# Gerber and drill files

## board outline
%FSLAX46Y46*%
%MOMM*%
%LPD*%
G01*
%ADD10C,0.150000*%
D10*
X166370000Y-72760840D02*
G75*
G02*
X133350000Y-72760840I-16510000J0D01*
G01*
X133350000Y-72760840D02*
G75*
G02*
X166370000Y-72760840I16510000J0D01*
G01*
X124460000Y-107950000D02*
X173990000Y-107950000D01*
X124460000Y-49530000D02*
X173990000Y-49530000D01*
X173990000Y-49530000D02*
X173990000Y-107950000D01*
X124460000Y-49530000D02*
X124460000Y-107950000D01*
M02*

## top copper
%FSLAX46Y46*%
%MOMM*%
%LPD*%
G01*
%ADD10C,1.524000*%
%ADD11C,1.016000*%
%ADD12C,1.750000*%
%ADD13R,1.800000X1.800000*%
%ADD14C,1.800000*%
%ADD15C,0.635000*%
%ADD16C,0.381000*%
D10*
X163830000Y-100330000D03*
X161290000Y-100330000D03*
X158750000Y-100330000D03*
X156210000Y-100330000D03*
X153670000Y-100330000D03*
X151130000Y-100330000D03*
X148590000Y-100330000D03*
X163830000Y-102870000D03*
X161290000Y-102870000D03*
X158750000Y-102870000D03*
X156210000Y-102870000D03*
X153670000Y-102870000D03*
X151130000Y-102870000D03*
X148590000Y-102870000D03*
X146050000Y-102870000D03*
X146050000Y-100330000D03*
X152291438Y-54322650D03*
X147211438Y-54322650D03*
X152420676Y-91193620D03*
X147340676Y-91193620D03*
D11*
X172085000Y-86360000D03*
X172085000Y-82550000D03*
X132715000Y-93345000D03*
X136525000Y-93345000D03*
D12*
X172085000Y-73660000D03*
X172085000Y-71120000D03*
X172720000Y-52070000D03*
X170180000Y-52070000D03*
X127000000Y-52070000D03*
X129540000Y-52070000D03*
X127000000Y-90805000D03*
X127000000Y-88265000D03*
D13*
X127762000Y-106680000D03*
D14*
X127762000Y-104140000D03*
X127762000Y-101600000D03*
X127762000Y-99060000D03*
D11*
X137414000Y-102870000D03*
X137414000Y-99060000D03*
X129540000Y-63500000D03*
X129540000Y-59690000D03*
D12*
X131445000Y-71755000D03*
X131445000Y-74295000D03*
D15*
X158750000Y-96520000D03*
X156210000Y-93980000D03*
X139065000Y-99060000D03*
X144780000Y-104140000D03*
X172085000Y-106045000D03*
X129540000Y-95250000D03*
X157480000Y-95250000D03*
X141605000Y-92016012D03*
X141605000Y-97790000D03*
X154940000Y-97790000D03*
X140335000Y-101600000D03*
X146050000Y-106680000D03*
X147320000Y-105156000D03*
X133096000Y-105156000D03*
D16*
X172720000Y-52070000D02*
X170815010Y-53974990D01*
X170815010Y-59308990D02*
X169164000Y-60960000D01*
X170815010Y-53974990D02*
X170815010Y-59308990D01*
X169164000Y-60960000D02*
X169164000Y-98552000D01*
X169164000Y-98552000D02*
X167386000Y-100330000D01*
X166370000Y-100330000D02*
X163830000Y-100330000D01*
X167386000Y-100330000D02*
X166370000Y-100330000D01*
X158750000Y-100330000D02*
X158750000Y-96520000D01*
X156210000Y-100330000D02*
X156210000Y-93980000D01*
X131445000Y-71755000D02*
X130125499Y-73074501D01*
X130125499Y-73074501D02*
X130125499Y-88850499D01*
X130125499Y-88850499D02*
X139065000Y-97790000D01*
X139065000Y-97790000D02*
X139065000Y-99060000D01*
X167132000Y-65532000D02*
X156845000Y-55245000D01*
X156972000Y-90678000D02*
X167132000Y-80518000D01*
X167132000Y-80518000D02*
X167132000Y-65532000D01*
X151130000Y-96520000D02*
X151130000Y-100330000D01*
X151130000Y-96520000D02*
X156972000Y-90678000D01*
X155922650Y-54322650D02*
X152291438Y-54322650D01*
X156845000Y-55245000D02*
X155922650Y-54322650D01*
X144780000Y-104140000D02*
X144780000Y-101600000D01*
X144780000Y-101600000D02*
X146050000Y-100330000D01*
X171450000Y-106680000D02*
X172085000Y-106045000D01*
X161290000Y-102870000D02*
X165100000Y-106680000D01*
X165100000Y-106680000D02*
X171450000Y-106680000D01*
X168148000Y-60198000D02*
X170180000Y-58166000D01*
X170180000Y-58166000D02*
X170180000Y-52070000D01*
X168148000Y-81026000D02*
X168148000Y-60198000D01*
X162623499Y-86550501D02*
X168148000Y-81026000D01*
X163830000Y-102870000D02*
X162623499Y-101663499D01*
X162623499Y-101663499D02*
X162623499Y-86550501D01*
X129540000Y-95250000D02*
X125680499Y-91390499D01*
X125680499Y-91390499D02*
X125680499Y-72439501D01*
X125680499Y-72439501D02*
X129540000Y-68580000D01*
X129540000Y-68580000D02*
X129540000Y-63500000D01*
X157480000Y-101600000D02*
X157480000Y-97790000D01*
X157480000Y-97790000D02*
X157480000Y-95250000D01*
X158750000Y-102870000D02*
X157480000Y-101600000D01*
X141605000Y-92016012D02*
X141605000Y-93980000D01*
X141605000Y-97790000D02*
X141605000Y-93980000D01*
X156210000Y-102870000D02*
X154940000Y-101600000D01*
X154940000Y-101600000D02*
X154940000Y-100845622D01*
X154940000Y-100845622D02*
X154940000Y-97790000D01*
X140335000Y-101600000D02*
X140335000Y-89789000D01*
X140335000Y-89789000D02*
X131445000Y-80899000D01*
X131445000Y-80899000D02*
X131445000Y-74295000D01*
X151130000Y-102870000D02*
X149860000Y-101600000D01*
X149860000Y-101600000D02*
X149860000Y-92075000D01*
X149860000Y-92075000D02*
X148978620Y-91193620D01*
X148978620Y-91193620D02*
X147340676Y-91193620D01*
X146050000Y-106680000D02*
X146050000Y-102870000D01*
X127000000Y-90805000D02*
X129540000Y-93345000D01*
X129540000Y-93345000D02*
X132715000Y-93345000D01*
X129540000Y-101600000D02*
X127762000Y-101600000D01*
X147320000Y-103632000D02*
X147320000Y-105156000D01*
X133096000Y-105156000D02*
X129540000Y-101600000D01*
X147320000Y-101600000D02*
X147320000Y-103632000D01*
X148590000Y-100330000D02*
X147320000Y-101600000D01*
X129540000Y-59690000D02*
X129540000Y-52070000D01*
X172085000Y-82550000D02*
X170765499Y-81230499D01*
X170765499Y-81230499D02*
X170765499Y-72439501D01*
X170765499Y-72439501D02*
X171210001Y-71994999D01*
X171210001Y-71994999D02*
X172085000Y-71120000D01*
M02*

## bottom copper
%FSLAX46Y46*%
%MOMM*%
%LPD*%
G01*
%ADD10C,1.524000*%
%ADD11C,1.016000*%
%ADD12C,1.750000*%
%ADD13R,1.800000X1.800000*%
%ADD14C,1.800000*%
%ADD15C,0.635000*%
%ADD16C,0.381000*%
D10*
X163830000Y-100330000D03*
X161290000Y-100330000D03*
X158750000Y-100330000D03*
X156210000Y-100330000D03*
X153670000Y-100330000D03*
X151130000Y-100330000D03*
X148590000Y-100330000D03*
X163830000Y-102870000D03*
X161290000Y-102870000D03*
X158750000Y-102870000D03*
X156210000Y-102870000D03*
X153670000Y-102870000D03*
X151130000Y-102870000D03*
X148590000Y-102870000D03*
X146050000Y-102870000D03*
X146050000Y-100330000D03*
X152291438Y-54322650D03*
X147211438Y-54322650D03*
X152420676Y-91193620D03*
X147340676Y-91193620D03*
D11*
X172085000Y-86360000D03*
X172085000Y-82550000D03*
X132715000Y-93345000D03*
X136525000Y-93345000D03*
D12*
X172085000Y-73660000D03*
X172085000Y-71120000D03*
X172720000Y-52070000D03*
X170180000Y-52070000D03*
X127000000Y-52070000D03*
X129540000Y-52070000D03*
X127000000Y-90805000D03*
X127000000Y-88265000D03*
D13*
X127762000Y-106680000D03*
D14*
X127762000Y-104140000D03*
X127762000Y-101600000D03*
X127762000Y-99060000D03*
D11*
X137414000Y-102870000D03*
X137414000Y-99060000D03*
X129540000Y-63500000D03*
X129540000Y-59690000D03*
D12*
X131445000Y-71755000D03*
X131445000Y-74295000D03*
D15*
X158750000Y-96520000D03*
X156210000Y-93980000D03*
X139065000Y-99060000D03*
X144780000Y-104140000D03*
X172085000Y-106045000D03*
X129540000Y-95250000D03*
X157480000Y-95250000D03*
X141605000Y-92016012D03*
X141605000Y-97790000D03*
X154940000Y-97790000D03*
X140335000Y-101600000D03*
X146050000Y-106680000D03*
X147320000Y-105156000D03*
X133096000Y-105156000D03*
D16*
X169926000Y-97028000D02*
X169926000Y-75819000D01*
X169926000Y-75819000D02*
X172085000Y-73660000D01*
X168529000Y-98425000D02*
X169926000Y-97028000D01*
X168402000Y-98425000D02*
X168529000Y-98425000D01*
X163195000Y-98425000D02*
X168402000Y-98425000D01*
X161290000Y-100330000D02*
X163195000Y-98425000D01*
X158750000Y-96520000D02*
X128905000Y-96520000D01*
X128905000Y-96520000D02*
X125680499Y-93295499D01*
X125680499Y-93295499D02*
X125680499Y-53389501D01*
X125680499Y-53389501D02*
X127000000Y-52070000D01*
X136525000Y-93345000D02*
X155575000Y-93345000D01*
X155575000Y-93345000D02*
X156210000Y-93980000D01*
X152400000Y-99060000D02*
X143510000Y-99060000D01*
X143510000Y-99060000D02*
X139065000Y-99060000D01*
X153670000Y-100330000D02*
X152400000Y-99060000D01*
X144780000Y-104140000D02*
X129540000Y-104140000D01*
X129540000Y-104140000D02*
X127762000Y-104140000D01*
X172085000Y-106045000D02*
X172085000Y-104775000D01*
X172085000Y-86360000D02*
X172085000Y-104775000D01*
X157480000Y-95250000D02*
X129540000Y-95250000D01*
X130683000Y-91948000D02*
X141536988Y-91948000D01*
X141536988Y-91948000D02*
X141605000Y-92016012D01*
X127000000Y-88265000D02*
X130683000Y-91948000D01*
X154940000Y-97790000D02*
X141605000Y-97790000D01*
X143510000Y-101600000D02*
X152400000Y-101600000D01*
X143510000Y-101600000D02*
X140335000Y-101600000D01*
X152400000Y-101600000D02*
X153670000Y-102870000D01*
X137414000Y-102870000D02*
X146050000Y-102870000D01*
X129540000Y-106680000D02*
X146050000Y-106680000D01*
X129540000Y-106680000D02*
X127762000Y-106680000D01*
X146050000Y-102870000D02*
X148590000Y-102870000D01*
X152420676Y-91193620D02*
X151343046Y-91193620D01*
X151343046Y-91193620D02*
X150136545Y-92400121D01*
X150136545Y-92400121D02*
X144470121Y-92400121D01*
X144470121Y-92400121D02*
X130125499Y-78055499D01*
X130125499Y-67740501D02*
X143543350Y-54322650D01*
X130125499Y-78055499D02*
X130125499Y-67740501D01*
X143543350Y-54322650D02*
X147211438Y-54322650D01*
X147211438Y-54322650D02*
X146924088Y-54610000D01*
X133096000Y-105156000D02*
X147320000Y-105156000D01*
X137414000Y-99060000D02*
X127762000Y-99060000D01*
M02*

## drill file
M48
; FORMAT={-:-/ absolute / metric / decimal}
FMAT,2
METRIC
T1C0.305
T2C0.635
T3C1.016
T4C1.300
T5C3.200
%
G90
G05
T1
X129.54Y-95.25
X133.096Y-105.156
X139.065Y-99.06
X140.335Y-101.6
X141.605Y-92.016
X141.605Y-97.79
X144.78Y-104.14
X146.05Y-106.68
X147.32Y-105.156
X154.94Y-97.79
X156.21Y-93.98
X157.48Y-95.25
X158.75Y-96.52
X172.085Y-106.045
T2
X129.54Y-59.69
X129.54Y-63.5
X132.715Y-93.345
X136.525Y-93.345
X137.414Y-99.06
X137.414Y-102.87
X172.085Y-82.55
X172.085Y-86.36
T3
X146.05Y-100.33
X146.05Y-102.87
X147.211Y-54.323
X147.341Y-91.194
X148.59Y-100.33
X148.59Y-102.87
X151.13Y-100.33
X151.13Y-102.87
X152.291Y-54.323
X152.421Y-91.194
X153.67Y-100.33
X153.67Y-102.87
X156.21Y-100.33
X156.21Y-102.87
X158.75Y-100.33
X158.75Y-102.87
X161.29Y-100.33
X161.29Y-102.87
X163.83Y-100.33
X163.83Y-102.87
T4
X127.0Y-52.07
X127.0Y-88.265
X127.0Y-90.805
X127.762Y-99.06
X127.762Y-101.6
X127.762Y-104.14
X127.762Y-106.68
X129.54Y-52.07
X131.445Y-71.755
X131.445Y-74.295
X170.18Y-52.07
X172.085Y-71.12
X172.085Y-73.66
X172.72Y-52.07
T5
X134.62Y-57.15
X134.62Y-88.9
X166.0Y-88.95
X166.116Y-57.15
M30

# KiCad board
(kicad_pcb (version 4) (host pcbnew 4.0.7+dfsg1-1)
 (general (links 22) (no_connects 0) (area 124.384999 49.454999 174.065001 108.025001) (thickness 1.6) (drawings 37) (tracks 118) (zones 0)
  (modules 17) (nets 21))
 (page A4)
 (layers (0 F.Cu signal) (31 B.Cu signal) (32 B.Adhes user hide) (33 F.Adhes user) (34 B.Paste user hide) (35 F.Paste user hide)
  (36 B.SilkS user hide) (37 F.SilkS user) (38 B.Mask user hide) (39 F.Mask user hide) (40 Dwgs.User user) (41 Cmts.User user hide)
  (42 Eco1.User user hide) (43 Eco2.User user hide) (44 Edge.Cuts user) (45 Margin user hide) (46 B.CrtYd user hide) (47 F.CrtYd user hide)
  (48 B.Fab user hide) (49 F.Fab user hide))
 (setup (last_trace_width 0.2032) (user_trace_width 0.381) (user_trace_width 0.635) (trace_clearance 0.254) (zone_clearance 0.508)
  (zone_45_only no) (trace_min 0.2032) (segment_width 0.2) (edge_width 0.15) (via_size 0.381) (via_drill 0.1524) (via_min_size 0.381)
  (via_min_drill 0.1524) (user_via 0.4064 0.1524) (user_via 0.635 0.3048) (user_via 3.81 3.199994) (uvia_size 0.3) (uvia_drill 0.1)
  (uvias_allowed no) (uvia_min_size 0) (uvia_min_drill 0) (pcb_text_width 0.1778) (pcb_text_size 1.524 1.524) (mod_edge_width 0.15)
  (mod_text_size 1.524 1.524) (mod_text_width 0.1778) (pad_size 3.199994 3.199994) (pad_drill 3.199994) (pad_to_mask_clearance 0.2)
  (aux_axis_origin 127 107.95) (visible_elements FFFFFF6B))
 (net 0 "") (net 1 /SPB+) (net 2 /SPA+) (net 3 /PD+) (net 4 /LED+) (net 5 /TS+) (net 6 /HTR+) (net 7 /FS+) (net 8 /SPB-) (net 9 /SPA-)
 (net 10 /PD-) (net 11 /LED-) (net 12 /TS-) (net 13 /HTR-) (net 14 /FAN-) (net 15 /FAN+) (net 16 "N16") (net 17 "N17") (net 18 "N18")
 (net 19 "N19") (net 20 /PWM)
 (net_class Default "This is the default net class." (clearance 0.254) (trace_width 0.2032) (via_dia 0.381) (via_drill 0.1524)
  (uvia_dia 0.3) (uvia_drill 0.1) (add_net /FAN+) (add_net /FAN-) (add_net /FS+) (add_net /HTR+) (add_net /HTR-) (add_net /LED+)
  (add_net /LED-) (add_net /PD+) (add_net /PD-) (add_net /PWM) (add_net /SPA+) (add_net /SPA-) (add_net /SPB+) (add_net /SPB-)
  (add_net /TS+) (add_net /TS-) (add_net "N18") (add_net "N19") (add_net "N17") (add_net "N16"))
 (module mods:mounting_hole (layer F.Cu) (at 166.116 57.15)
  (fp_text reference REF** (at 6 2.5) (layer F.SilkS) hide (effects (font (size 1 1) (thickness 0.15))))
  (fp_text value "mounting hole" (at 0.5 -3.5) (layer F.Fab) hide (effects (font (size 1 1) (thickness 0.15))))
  (pad "" np_thru_hole circle (at 0 0) (size 3.199994 3.199994) (drill 3.199994) (layers *.Cu *.Mask F.SilkS)))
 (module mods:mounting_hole (layer F.Cu) (at 134.62 88.9)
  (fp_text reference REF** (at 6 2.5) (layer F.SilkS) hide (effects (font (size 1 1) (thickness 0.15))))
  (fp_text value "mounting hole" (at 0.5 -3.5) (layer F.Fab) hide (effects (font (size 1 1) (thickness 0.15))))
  (pad "" np_thru_hole circle (at 0 0) (size 3.199994 3.199994) (drill 3.199994) (layers *.Cu *.Mask F.SilkS)))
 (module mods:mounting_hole (layer F.Cu) (at 134.62 57.15)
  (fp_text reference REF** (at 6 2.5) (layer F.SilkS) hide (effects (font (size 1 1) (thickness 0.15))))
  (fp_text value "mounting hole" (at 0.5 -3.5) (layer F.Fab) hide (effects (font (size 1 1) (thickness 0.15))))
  (pad "" np_thru_hole circle (at 0 0) (size 3.199994 3.199994) (drill 3.199994) (layers *.Cu *.Mask F.SilkS)))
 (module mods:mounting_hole (layer F.Cu) (at 165.999998 88.950013)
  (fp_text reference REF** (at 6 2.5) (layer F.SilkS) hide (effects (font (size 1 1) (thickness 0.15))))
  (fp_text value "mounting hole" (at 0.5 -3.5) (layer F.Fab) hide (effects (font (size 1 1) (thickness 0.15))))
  (pad "" np_thru_hole circle (at 0 0) (size 3.199994 3.199994) (drill 3.199994) (layers *.Cu *.Mask F.SilkS)))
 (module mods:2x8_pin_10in (layer F.Cu) (at 154.94 101.6 180)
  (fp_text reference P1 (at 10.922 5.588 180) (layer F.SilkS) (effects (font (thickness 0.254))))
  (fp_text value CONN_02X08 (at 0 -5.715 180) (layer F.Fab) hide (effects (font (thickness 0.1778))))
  (pad 1 thru_hole circle (at -8.89 1.27 180) (size 1.524 1.524) (drill 1.016) (layers *.Cu *.Mask F.SilkS) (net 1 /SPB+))
  (pad 3 thru_hole circle (at -6.35 1.27 180) (size 1.524 1.524) (drill 1.016) (layers *.Cu *.Mask F.SilkS) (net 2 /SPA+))
  (pad 5 thru_hole circle (at -3.81 1.27 180) (size 1.524 1.524) (drill 1.016) (layers *.Cu *.Mask F.SilkS) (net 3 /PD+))
  (pad 7 thru_hole circle (at -1.27 1.27 180) (size 1.524 1.524) (drill 1.016) (layers *.Cu *.Mask F.SilkS) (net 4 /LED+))
  (pad 9 thru_hole circle (at 1.27 1.27 180) (size 1.524 1.524) (drill 1.016) (layers *.Cu *.Mask F.SilkS) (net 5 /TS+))
  (pad 11 thru_hole circle (at 3.81 1.27 180) (size 1.524 1.524) (drill 1.016) (layers *.Cu *.Mask F.SilkS) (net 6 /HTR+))
  (pad 13 thru_hole circle (at 6.35 1.27 180) (size 1.524 1.524) (drill 1.016) (layers *.Cu *.Mask F.SilkS) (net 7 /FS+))
  (pad 2 thru_hole circle (at -8.89 -1.27 180) (size 1.524 1.524) (drill 1.016) (layers *.Cu *.Mask F.SilkS) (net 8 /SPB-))
  (pad 4 thru_hole circle (at -6.35 -1.27 180) (size 1.524 1.524) (drill 1.016) (layers *.Cu *.Mask F.SilkS) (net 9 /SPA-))
  (pad 6 thru_hole circle (at -3.81 -1.27 180) (size 1.524 1.524) (drill 1.016) (layers *.Cu *.Mask F.SilkS) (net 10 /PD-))
  (pad 8 thru_hole circle (at -1.27 -1.27 180) (size 1.524 1.524) (drill 1.016) (layers *.Cu *.Mask F.SilkS) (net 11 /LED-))
  (pad 10 thru_hole circle (at 1.27 -1.27 180) (size 1.524 1.524) (drill 1.016) (layers *.Cu *.Mask F.SilkS) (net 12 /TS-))
  (pad 12 thru_hole circle (at 3.81 -1.27 180) (size 1.524 1.524) (drill 1.016) (layers *.Cu *.Mask F.SilkS) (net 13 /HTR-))
  (pad 14 thru_hole circle (at 6.35 -1.27 180) (size 1.524 1.524) (drill 1.016) (layers *.Cu *.Mask F.SilkS) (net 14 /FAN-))
  (pad 16 thru_hole circle (at 8.89 -1.27 180) (size 1.524 1.524) (drill 1.016) (layers *.Cu *.Mask F.SilkS) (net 14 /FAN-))
  (pad 15 thru_hole circle (at 8.89 1.27 180) (size 1.524 1.524) (drill 1.016) (layers *.Cu *.Mask F.SilkS) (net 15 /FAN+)))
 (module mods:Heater (layer F.Cu) (at 149.751438 54.32265 180)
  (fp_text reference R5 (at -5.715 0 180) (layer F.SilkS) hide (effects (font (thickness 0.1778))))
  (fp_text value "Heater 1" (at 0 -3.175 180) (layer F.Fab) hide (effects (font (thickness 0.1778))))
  (pad 1 thru_hole circle (at -2.54 0 180) (size 1.524 1.524) (drill 1.016) (layers *.Cu *.Mask F.SilkS) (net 6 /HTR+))
  (pad 2 thru_hole circle (at 2.54 0 180) (size 1.524 1.524) (drill 1.016) (layers *.Cu *.Mask F.SilkS) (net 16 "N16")))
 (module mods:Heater (layer F.Cu) (at 149.880676 91.19362 180)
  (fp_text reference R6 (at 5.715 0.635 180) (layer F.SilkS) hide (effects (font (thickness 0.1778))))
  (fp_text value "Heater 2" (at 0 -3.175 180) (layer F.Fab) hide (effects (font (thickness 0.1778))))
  (pad 1 thru_hole circle (at -2.54 0 180) (size 1.524 1.524) (drill 1.016) (layers *.Cu *.Mask F.SilkS) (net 16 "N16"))
  (pad 2 thru_hole circle (at 2.54 0 180) (size 1.524 1.524) (drill 1.016) (layers *.Cu *.Mask F.SilkS) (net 13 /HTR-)))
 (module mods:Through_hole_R (layer F.Cu) (at 172.085 84.455 90)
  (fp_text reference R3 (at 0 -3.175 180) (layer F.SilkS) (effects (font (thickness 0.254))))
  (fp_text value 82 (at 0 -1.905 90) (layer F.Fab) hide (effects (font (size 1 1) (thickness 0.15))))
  (pad 2 thru_hole circle (at -1.905 0 90) (size 1.016 1.016) (drill 0.635) (layers *.Cu *.Mask F.SilkS) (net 9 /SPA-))
  (pad 1 thru_hole circle (at 1.905 0 90) (size 1.016 1.016) (drill 0.635) (layers *.Cu *.Mask F.SilkS) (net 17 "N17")))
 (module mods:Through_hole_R (layer F.Cu) (at 134.62 93.345)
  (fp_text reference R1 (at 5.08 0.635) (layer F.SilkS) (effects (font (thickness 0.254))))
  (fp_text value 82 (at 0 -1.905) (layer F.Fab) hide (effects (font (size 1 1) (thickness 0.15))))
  (pad 2 thru_hole circle (at -1.905 0) (size 1.016 1.016) (drill 0.635) (layers *.Cu *.Mask F.SilkS) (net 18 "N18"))
  (pad 1 thru_hole circle (at 1.905 0) (size 1.016 1.016) (drill 0.635) (layers *.Cu *.Mask F.SilkS) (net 4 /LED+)))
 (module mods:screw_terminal (layer F.Cu) (at 172.085 72.39 90)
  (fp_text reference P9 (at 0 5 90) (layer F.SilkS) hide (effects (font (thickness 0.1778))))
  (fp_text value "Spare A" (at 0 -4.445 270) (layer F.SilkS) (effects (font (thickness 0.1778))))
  (pad 1 thru_hole circle (at -1.27 0 90) (size 1.75 1.75) (drill 1.3) (layers *.Cu *.Mask F.SilkS) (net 2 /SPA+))
  (pad 2 thru_hole circle (at 1.27 0 90) (size 1.75 1.75) (drill 1.3) (layers *.Cu *.Mask F.SilkS) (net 17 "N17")))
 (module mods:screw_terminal (layer F.Cu) (at 171.45 52.07 180)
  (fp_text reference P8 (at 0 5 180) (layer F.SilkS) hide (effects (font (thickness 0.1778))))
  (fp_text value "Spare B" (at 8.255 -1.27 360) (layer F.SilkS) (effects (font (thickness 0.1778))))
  (pad 1 thru_hole circle (at -1.27 0 180) (size 1.75 1.75) (drill 1.3) (layers *.Cu *.Mask F.SilkS) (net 1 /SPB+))
  (pad 2 thru_hole circle (at 1.27 0 180) (size 1.75 1.75) (drill 1.3) (layers *.Cu *.Mask F.SilkS) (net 8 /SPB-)))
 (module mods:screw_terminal (layer F.Cu) (at 128.27 52.07)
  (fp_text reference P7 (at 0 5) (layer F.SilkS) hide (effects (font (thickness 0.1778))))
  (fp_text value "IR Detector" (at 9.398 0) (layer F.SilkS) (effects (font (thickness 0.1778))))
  (pad 1 thru_hole circle (at -1.27 0) (size 1.75 1.75) (drill 1.3) (layers *.Cu *.Mask F.SilkS) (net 3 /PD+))
  (pad 2 thru_hole circle (at 1.27 0) (size 1.75 1.75) (drill 1.3) (layers *.Cu *.Mask F.SilkS) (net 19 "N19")))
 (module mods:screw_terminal (layer F.Cu) (at 127 89.535 90)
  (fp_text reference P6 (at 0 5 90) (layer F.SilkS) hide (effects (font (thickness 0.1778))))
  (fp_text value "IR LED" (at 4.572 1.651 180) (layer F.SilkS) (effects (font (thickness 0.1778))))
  (pad 1 thru_hole circle (at -1.27 0 90) (size 1.75 1.75) (drill 1.3) (layers *.Cu *.Mask F.SilkS) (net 18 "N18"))
  (pad 2 thru_hole circle (at 1.27 0 90) (size 1.75 1.75) (drill 1.3) (layers *.Cu *.Mask F.SilkS) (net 11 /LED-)))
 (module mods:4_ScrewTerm (layer F.Cu) (at 127.762 102.87 90)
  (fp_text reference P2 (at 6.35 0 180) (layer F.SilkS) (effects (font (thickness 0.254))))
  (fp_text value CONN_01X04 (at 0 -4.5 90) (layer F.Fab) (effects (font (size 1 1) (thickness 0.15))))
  (pad 1 thru_hole rect (at -3.81 0 90) (size 1.8 1.8) (drill 1.3) (layers *.Cu *.Mask) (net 14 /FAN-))
  (pad 2 thru_hole circle (at -1.27 0 90) (size 1.8 1.8) (drill 1.3) (layers *.Cu *.Mask) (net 15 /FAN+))
  (pad 3 thru_hole circle (at 1.27 0 90) (size 1.8 1.8) (drill 1.3) (layers *.Cu *.Mask) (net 7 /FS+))
  (pad 4 thru_hole circle (at 3.81 0 90) (size 1.8 1.8) (drill 1.3) (layers *.Cu *.Mask) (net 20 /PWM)))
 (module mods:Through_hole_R (layer F.Cu) (at 137.414 100.965 90)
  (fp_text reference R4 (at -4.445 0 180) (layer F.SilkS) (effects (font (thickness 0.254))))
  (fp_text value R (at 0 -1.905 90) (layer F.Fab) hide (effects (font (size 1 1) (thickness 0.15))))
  (pad 2 thru_hole circle (at -1.905 0 90) (size 1.016 1.016) (drill 0.635) (layers *.Cu *.Mask F.SilkS) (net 14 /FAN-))
  (pad 1 thru_hole circle (at 1.905 0 90) (size 1.016 1.016) (drill 0.635) (layers *.Cu *.Mask F.SilkS) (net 20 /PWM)))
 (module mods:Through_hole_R (layer F.Cu) (at 129.54 61.595 90)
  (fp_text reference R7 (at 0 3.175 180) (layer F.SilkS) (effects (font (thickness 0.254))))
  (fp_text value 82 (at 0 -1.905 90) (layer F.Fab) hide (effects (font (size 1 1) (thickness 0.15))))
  (pad 2 thru_hole circle (at -1.905 0 90) (size 1.016 1.016) (drill 0.635) (layers *.Cu *.Mask F.SilkS) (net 10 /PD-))
  (pad 1 thru_hole circle (at 1.905 0 90) (size 1.016 1.016) (drill 0.635) (layers *.Cu *.Mask F.SilkS) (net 19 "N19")))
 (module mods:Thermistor (layer F.Cu) (at 131.445 73.025 270)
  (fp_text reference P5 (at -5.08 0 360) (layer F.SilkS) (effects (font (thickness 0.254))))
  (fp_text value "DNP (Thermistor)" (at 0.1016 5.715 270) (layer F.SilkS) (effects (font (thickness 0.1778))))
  (pad 1 thru_hole circle (at -1.27 0 270) (size 1.75 1.75) (drill 1.3) (layers *.Cu *.Mask F.SilkS) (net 5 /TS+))
  (pad 2 thru_hole circle (at 1.27 0 270) (size 1.75 1.75) (drill 1.3) (layers *.Cu *.Mask F.SilkS) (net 12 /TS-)))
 (gr_circle (center 149.86 72.76084) (end 133.35 72.76084) (layer Edge.Cuts) (width 0.15))
 (gr_line (start 124.46 107.95) (end 173.99 107.95) (angle 90) (layer Edge.Cuts) (width 0.15))
 (gr_line (start 124.46 49.53) (end 173.99 49.53) (angle 90) (layer Edge.Cuts) (width 0.15))
 (gr_line (start 173.99 49.53) (end 173.99 107.95) (angle 90) (layer Edge.Cuts) (width 0.15))
 (gr_line (start 124.46 49.53) (end 124.46 107.95) (angle 90) (layer Edge.Cuts) (width 0.15))
 (segment (start 169.926 97.028) (end 169.926 75.819) (width 0.381) (layer B.Cu) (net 2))
 (segment (start 169.926 75.819) (end 172.085 73.66) (width 0.381) (layer B.Cu) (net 2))
 (segment (start 168.529 98.425) (end 169.926 97.028) (width 0.381) (layer B.Cu) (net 2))
 (segment (start 168.402 98.425) (end 168.529 98.425) (width 0.381) (layer B.Cu) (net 2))
 (segment (start 163.195 98.425) (end 168.402 98.425) (width 0.381) (layer B.Cu) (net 2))
 (segment (start 161.29 100.33) (end 163.195 98.425) (width 0.381) (layer B.Cu) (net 2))
 (segment (start 172.72 52.07) (end 170.81501 53.97499) (width 0.381) (layer F.Cu) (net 1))
 (segment (start 170.81501 59.30899) (end 169.164 60.96) (width 0.381) (layer F.Cu) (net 1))
 (segment (start 170.81501 53.97499) (end 170.81501 59.30899) (width 0.381) (layer F.Cu) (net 1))
 (segment (start 169.164 60.96) (end 169.164 98.552) (width 0.381) (layer F.Cu) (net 1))
 (segment (start 169.164 98.552) (end 167.386 100.33) (width 0.381) (layer F.Cu) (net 1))
 (segment (start 166.37 100.33) (end 163.83 100.33) (width 0.381) (layer F.Cu) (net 1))
 (segment (start 167.386 100.33) (end 166.37 100.33) (width 0.381) (layer F.Cu) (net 1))
 (segment (start 158.75 96.52) (end 128.905 96.52) (width 0.381) (layer B.Cu) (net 3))
 (segment (start 128.905 96.52) (end 125.680499 93.295499) (width 0.381) (layer B.Cu) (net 3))
 (segment (start 125.680499 93.295499) (end 125.680499 53.389501) (width 0.381) (layer B.Cu) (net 3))
 (segment (start 125.680499 53.389501) (end 127 52.07) (width 0.381) (layer B.Cu) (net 3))
 (via (at 158.75 96.52) (size 0.635) (drill 0.3048) (layers F.Cu B.Cu) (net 3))
 (segment (start 158.75 100.33) (end 158.75 96.52) (width 0.381) (layer F.Cu) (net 3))
 (segment (start 136.525 93.345) (end 155.575 93.345) (width 0.381) (layer B.Cu) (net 4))
 (segment (start 155.575 93.345) (end 156.21 93.98) (width 0.381) (layer B.Cu) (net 4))
 (via (at 156.21 93.98) (size 0.635) (drill 0.3048) (layers F.Cu B.Cu) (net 4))
 (segment (start 156.21 100.33) (end 156.21 93.98) (width 0.381) (layer F.Cu) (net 4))
 (segment (start 131.445 71.755) (end 130.125499 73.074501) (width 0.381) (layer F.Cu) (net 5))
 (segment (start 130.125499 73.074501) (end 130.125499 88.850499) (width 0.381) (layer F.Cu) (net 5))
 (segment (start 130.125499 88.850499) (end 139.065 97.79) (width 0.381) (layer F.Cu) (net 5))
 (segment (start 139.065 97.79) (end 139.065 99.06) (width 0.381) (layer F.Cu) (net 5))
 (via (at 139.065 99.06) (size 0.635) (drill 0.3048) (layers F.Cu B.Cu) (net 5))
 (segment (start 152.4 99.06) (end 143.51 99.06) (width 0.381) (layer B.Cu) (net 5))
 (segment (start 143.51 99.06) (end 139.065 99.06) (width 0.381) (layer B.Cu) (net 5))
 (segment (start 153.67 100.33) (end 152.4 99.06) (width 0.381) (layer B.Cu) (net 5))
 (segment (start 167.132 65.532) (end 156.845 55.245) (width 0.381) (layer F.Cu) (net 6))
 (segment (start 156.972 90.678) (end 167.132 80.518) (width 0.381) (layer F.Cu) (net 6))
 (segment (start 167.132 80.518) (end 167.132 65.532) (width 0.381) (layer F.Cu) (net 6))
 (segment (start 151.13 96.52) (end 151.13 100.33) (width 0.381) (layer F.Cu) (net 6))
 (segment (start 151.13 96.52) (end 156.972 90.678) (width 0.381) (layer F.Cu) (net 6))
 (segment (start 155.92265 54.32265) (end 152.291438 54.32265) (width 0.381) (layer F.Cu) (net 6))
 (segment (start 156.845 55.245) (end 155.92265 54.32265) (width 0.381) (layer F.Cu) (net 6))
 (segment (start 144.78 104.14) (end 129.54 104.14) (width 0.381) (layer B.Cu) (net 15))
 (segment (start 129.54 104.14) (end 127.762 104.14) (width 0.381) (layer B.Cu) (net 15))
 (segment (start 144.78 104.14) (end 144.78 101.6) (width 0.381) (layer F.Cu) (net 15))
 (segment (start 144.78 101.6) (end 146.05 100.33) (width 0.381) (layer F.Cu) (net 15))
 (via (at 144.78 104.14) (size 0.635) (drill 0.3048) (layers F.Cu B.Cu) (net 15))
 (segment (start 172.085 106.045) (end 172.085 104.775) (width 0.381) (layer B.Cu) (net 9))
 (segment (start 171.45 106.68) (end 172.085 106.045) (width 0.381) (layer F.Cu) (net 9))
 (via (at 172.085 106.045) (size 0.635) (drill 0.3048) (layers F.Cu B.Cu) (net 9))
 (segment (start 161.29 102.87) (end 165.1 106.68) (width 0.381) (layer F.Cu) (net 9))
 (segment (start 165.1 106.68) (end 171.45 106.68) (width 0.381) (layer F.Cu) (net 9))
 (segment (start 172.085 86.36) (end 172.085 104.775) (width 0.381) (layer B.Cu) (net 9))
 (segment (start 168.148 60.198) (end 170.18 58.166) (width 0.381) (layer F.Cu) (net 8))
 (segment (start 170.18 58.166) (end 170.18 52.07) (width 0.381) (layer F.Cu) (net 8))
 (segment (start 168.148 81.026) (end 168.148 60.198) (width 0.381) (layer F.Cu) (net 8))
 (segment (start 162.623499 86.550501) (end 168.148 81.026) (width 0.381) (layer F.Cu) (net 8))
 (segment (start 163.83 102.87) (end 162.623499 101.663499) (width 0.381) (layer F.Cu) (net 8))
 (segment (start 162.623499 101.663499) (end 162.623499 86.550501) (width 0.381) (layer F.Cu) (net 8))
 (segment (start 129.54 95.25) (end 125.680499 91.390499) (width 0.381) (layer F.Cu) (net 10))
 (segment (start 125.680499 91.390499) (end 125.680499 72.439501) (width 0.381) (layer F.Cu) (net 10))
 (segment (start 125.680499 72.439501) (end 129.54 68.58) (width 0.381) (layer F.Cu) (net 10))
 (segment (start 129.54 68.58) (end 129.54 63.5) (width 0.381) (layer F.Cu) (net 10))
 (segment (start 157.48 95.25) (end 129.54 95.25) (width 0.381) (layer B.Cu) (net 10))
 (via (at 129.54 95.25) (size 0.635) (drill 0.3048) (layers F.Cu B.Cu) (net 10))
 (segment (start 157.48 101.6) (end 157.48 97.79) (width 0.381) (layer F.Cu) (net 10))
 (segment (start 157.48 97.79) (end 157.48 95.25) (width 0.381) (layer F.Cu) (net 10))
 (via (at 157.48 95.25) (size 0.635) (drill 0.3048) (layers F.Cu B.Cu) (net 10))
 (segment (start 158.75 102.87) (end 157.48 101.6) (width 0.381) (layer F.Cu) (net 10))
 (segment (start 141.605 92.016012) (end 141.605 93.98) (width 0.381) (layer F.Cu) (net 11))
 (segment (start 130.683 91.948) (end 141.536988 91.948) (width 0.381) (layer B.Cu) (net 11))
 (segment (start 141.536988 91.948) (end 141.605 92.016012) (width 0.381) (layer B.Cu) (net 11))
 (via (at 141.605 92.016012) (size 0.635) (drill 0.3048) (layers F.Cu B.Cu) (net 11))
 (segment (start 127 88.265) (end 130.683 91.948) (width 0.381) (layer B.Cu) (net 11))
 (segment (start 141.605 97.79) (end 141.605 93.98) (width 0.381) (layer F.Cu) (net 11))
 (segment (start 154.94 97.79) (end 141.605 97.79) (width 0.381) (layer B.Cu) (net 11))
 (via (at 141.605 97.79) (size 0.635) (drill 0.3048) (layers F.Cu B.Cu) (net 11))
 (segment (start 156.21 102.87) (end 154.94 101.6) (width 0.381) (layer F.Cu) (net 11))
 (segment (start 154.94 101.6) (end 154.94 100.845622) (width 0.381) (layer F.Cu) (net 11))
 (segment (start 154.94 100.845622) (end 154.94 97.79) (width 0.381) (layer F.Cu) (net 11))
 (via (at 154.94 97.79) (size 0.635) (drill 0.3048) (layers F.Cu B.Cu) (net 11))
 (segment (start 140.335 101.6) (end 140.335 89.789) (width 0.381) (layer F.Cu) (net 12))
 (segment (start 140.335 89.789) (end 131.445 80.899) (width 0.381) (layer F.Cu) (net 12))
 (segment (start 131.445 80.899) (end 131.445 74.295) (width 0.381) (layer F.Cu) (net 12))
 (segment (start 143.51 101.6) (end 152.4 101.6) (width 0.381) (layer B.Cu) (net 12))
 (segment (start 143.51 101.6) (end 140.335 101.6) (width 0.381) (layer B.Cu) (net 12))
 (via (at 140.335 101.6) (size 0.635) (drill 0.3048) (layers F.Cu B.Cu) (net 12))
 (segment (start 152.4 101.6) (end 153.67 102.87) (width 0.381) (layer B.Cu) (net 12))
 (segment (start 151.13 102.87) (end 149.86 101.6) (width 0.381) (layer F.Cu) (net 13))
 (segment (start 149.86 101.6) (end 149.86 92.075) (width 0.381) (layer F.Cu) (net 13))
 (segment (start 149.86 92.075) (end 148.97862 91.19362) (width 0.381) (layer F.Cu) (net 13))
 (segment (start 148.97862 91.19362) (end 147.340676 91.19362) (width 0.381) (layer F.Cu) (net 13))
 (segment (start 137.414 102.87) (end 146.05 102.87) (width 0.381) (layer B.Cu) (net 14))
 (segment (start 146.05 106.68) (end 146.05 102.87) (width 0.381) (layer F.Cu) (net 14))
 (segment (start 129.54 106.68) (end 146.05 106.68) (width 0.381) (layer B.Cu) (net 14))
 (via (at 146.05 106.68) (size 0.635) (drill 0.3048) (layers F.Cu B.Cu) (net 14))
 (segment (start 129.54 106.68) (end 127.762 106.68) (width 0.381) (layer B.Cu) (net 14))
 (segment (start 146.05 102.87) (end 148.59 102.87) (width 0.381) (layer B.Cu) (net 14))
 (segment (start 127 90.805) (end 129.54 93.345) (width 0.381) (layer F.Cu) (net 18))
 (segment (start 129.54 93.345) (end 132.715 93.345) (width 0.381) (layer F.Cu) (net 18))
 (segment (start 152.420676 91.19362) (end 151.343046 91.19362) (width 0.381) (layer B.Cu) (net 16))
 (segment (start 151.343046 91.19362) (end 150.136545 92.400121) (width 0.381) (layer B.Cu) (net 16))
 (segment (start 150.136545 92.400121) (end 144.470121 92.400121) (width 0.381) (layer B.Cu) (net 16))
 (segment (start 144.470121 92.400121) (end 130.125499 78.055499) (width 0.381) (layer B.Cu) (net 16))
 (segment (start 130.125499 67.740501) (end 143.54335 54.32265) (width 0.381) (layer B.Cu) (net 16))
 (segment (start 130.125499 78.055499) (end 130.125499 67.740501) (width 0.381) (layer B.Cu) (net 16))
 (segment (start 143.54335 54.32265) (end 147.211438 54.32265) (width 0.381) (layer B.Cu) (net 16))
 (segment (start 147.211438 54.32265) (end 146.924088 54.61) (width 0.381) (layer B.Cu) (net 16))
 (segment (start 129.54 101.6) (end 127.762 101.6) (width 0.381) (layer F.Cu) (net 7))
 (segment (start 147.32 103.632) (end 147.32 105.156) (width 0.381) (layer F.Cu) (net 7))
 (segment (start 133.096 105.156) (end 147.32 105.156) (width 0.381) (layer B.Cu) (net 7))
 (via (at 147.32 105.156) (size 0.635) (drill 0.3048) (layers F.Cu B.Cu) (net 7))
 (segment (start 133.096 105.156) (end 129.54 101.6) (width 0.381) (layer F.Cu) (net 7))
 (via (at 133.096 105.156) (size 0.635) (drill 0.3048) (layers F.Cu B.Cu) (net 7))
 (segment (start 147.32 101.6) (end 147.32 103.632) (width 0.381) (layer F.Cu) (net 7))
 (segment (start 148.59 100.33) (end 147.32 101.6) (width 0.381) (layer F.Cu) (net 7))
 (segment (start 137.414 99.06) (end 127.762 99.06) (width 0.381) (layer B.Cu) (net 20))
 (segment (start 129.54 59.69) (end 129.54 52.07) (width 0.381) (layer F.Cu) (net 19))
 (segment (start 172.085 82.55) (end 170.765499 81.230499) (width 0.381) (layer F.Cu) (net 17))
 (segment (start 170.765499 81.230499) (end 170.765499 72.439501) (width 0.381) (layer F.Cu) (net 17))
 (segment (start 170.765499 72.439501) (end 171.210001 71.994999) (width 0.381) (layer F.Cu) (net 17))
 (segment (start 171.210001 71.994999) (end 172.085 71.12) (width 0.381) (layer F.Cu) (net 17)))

